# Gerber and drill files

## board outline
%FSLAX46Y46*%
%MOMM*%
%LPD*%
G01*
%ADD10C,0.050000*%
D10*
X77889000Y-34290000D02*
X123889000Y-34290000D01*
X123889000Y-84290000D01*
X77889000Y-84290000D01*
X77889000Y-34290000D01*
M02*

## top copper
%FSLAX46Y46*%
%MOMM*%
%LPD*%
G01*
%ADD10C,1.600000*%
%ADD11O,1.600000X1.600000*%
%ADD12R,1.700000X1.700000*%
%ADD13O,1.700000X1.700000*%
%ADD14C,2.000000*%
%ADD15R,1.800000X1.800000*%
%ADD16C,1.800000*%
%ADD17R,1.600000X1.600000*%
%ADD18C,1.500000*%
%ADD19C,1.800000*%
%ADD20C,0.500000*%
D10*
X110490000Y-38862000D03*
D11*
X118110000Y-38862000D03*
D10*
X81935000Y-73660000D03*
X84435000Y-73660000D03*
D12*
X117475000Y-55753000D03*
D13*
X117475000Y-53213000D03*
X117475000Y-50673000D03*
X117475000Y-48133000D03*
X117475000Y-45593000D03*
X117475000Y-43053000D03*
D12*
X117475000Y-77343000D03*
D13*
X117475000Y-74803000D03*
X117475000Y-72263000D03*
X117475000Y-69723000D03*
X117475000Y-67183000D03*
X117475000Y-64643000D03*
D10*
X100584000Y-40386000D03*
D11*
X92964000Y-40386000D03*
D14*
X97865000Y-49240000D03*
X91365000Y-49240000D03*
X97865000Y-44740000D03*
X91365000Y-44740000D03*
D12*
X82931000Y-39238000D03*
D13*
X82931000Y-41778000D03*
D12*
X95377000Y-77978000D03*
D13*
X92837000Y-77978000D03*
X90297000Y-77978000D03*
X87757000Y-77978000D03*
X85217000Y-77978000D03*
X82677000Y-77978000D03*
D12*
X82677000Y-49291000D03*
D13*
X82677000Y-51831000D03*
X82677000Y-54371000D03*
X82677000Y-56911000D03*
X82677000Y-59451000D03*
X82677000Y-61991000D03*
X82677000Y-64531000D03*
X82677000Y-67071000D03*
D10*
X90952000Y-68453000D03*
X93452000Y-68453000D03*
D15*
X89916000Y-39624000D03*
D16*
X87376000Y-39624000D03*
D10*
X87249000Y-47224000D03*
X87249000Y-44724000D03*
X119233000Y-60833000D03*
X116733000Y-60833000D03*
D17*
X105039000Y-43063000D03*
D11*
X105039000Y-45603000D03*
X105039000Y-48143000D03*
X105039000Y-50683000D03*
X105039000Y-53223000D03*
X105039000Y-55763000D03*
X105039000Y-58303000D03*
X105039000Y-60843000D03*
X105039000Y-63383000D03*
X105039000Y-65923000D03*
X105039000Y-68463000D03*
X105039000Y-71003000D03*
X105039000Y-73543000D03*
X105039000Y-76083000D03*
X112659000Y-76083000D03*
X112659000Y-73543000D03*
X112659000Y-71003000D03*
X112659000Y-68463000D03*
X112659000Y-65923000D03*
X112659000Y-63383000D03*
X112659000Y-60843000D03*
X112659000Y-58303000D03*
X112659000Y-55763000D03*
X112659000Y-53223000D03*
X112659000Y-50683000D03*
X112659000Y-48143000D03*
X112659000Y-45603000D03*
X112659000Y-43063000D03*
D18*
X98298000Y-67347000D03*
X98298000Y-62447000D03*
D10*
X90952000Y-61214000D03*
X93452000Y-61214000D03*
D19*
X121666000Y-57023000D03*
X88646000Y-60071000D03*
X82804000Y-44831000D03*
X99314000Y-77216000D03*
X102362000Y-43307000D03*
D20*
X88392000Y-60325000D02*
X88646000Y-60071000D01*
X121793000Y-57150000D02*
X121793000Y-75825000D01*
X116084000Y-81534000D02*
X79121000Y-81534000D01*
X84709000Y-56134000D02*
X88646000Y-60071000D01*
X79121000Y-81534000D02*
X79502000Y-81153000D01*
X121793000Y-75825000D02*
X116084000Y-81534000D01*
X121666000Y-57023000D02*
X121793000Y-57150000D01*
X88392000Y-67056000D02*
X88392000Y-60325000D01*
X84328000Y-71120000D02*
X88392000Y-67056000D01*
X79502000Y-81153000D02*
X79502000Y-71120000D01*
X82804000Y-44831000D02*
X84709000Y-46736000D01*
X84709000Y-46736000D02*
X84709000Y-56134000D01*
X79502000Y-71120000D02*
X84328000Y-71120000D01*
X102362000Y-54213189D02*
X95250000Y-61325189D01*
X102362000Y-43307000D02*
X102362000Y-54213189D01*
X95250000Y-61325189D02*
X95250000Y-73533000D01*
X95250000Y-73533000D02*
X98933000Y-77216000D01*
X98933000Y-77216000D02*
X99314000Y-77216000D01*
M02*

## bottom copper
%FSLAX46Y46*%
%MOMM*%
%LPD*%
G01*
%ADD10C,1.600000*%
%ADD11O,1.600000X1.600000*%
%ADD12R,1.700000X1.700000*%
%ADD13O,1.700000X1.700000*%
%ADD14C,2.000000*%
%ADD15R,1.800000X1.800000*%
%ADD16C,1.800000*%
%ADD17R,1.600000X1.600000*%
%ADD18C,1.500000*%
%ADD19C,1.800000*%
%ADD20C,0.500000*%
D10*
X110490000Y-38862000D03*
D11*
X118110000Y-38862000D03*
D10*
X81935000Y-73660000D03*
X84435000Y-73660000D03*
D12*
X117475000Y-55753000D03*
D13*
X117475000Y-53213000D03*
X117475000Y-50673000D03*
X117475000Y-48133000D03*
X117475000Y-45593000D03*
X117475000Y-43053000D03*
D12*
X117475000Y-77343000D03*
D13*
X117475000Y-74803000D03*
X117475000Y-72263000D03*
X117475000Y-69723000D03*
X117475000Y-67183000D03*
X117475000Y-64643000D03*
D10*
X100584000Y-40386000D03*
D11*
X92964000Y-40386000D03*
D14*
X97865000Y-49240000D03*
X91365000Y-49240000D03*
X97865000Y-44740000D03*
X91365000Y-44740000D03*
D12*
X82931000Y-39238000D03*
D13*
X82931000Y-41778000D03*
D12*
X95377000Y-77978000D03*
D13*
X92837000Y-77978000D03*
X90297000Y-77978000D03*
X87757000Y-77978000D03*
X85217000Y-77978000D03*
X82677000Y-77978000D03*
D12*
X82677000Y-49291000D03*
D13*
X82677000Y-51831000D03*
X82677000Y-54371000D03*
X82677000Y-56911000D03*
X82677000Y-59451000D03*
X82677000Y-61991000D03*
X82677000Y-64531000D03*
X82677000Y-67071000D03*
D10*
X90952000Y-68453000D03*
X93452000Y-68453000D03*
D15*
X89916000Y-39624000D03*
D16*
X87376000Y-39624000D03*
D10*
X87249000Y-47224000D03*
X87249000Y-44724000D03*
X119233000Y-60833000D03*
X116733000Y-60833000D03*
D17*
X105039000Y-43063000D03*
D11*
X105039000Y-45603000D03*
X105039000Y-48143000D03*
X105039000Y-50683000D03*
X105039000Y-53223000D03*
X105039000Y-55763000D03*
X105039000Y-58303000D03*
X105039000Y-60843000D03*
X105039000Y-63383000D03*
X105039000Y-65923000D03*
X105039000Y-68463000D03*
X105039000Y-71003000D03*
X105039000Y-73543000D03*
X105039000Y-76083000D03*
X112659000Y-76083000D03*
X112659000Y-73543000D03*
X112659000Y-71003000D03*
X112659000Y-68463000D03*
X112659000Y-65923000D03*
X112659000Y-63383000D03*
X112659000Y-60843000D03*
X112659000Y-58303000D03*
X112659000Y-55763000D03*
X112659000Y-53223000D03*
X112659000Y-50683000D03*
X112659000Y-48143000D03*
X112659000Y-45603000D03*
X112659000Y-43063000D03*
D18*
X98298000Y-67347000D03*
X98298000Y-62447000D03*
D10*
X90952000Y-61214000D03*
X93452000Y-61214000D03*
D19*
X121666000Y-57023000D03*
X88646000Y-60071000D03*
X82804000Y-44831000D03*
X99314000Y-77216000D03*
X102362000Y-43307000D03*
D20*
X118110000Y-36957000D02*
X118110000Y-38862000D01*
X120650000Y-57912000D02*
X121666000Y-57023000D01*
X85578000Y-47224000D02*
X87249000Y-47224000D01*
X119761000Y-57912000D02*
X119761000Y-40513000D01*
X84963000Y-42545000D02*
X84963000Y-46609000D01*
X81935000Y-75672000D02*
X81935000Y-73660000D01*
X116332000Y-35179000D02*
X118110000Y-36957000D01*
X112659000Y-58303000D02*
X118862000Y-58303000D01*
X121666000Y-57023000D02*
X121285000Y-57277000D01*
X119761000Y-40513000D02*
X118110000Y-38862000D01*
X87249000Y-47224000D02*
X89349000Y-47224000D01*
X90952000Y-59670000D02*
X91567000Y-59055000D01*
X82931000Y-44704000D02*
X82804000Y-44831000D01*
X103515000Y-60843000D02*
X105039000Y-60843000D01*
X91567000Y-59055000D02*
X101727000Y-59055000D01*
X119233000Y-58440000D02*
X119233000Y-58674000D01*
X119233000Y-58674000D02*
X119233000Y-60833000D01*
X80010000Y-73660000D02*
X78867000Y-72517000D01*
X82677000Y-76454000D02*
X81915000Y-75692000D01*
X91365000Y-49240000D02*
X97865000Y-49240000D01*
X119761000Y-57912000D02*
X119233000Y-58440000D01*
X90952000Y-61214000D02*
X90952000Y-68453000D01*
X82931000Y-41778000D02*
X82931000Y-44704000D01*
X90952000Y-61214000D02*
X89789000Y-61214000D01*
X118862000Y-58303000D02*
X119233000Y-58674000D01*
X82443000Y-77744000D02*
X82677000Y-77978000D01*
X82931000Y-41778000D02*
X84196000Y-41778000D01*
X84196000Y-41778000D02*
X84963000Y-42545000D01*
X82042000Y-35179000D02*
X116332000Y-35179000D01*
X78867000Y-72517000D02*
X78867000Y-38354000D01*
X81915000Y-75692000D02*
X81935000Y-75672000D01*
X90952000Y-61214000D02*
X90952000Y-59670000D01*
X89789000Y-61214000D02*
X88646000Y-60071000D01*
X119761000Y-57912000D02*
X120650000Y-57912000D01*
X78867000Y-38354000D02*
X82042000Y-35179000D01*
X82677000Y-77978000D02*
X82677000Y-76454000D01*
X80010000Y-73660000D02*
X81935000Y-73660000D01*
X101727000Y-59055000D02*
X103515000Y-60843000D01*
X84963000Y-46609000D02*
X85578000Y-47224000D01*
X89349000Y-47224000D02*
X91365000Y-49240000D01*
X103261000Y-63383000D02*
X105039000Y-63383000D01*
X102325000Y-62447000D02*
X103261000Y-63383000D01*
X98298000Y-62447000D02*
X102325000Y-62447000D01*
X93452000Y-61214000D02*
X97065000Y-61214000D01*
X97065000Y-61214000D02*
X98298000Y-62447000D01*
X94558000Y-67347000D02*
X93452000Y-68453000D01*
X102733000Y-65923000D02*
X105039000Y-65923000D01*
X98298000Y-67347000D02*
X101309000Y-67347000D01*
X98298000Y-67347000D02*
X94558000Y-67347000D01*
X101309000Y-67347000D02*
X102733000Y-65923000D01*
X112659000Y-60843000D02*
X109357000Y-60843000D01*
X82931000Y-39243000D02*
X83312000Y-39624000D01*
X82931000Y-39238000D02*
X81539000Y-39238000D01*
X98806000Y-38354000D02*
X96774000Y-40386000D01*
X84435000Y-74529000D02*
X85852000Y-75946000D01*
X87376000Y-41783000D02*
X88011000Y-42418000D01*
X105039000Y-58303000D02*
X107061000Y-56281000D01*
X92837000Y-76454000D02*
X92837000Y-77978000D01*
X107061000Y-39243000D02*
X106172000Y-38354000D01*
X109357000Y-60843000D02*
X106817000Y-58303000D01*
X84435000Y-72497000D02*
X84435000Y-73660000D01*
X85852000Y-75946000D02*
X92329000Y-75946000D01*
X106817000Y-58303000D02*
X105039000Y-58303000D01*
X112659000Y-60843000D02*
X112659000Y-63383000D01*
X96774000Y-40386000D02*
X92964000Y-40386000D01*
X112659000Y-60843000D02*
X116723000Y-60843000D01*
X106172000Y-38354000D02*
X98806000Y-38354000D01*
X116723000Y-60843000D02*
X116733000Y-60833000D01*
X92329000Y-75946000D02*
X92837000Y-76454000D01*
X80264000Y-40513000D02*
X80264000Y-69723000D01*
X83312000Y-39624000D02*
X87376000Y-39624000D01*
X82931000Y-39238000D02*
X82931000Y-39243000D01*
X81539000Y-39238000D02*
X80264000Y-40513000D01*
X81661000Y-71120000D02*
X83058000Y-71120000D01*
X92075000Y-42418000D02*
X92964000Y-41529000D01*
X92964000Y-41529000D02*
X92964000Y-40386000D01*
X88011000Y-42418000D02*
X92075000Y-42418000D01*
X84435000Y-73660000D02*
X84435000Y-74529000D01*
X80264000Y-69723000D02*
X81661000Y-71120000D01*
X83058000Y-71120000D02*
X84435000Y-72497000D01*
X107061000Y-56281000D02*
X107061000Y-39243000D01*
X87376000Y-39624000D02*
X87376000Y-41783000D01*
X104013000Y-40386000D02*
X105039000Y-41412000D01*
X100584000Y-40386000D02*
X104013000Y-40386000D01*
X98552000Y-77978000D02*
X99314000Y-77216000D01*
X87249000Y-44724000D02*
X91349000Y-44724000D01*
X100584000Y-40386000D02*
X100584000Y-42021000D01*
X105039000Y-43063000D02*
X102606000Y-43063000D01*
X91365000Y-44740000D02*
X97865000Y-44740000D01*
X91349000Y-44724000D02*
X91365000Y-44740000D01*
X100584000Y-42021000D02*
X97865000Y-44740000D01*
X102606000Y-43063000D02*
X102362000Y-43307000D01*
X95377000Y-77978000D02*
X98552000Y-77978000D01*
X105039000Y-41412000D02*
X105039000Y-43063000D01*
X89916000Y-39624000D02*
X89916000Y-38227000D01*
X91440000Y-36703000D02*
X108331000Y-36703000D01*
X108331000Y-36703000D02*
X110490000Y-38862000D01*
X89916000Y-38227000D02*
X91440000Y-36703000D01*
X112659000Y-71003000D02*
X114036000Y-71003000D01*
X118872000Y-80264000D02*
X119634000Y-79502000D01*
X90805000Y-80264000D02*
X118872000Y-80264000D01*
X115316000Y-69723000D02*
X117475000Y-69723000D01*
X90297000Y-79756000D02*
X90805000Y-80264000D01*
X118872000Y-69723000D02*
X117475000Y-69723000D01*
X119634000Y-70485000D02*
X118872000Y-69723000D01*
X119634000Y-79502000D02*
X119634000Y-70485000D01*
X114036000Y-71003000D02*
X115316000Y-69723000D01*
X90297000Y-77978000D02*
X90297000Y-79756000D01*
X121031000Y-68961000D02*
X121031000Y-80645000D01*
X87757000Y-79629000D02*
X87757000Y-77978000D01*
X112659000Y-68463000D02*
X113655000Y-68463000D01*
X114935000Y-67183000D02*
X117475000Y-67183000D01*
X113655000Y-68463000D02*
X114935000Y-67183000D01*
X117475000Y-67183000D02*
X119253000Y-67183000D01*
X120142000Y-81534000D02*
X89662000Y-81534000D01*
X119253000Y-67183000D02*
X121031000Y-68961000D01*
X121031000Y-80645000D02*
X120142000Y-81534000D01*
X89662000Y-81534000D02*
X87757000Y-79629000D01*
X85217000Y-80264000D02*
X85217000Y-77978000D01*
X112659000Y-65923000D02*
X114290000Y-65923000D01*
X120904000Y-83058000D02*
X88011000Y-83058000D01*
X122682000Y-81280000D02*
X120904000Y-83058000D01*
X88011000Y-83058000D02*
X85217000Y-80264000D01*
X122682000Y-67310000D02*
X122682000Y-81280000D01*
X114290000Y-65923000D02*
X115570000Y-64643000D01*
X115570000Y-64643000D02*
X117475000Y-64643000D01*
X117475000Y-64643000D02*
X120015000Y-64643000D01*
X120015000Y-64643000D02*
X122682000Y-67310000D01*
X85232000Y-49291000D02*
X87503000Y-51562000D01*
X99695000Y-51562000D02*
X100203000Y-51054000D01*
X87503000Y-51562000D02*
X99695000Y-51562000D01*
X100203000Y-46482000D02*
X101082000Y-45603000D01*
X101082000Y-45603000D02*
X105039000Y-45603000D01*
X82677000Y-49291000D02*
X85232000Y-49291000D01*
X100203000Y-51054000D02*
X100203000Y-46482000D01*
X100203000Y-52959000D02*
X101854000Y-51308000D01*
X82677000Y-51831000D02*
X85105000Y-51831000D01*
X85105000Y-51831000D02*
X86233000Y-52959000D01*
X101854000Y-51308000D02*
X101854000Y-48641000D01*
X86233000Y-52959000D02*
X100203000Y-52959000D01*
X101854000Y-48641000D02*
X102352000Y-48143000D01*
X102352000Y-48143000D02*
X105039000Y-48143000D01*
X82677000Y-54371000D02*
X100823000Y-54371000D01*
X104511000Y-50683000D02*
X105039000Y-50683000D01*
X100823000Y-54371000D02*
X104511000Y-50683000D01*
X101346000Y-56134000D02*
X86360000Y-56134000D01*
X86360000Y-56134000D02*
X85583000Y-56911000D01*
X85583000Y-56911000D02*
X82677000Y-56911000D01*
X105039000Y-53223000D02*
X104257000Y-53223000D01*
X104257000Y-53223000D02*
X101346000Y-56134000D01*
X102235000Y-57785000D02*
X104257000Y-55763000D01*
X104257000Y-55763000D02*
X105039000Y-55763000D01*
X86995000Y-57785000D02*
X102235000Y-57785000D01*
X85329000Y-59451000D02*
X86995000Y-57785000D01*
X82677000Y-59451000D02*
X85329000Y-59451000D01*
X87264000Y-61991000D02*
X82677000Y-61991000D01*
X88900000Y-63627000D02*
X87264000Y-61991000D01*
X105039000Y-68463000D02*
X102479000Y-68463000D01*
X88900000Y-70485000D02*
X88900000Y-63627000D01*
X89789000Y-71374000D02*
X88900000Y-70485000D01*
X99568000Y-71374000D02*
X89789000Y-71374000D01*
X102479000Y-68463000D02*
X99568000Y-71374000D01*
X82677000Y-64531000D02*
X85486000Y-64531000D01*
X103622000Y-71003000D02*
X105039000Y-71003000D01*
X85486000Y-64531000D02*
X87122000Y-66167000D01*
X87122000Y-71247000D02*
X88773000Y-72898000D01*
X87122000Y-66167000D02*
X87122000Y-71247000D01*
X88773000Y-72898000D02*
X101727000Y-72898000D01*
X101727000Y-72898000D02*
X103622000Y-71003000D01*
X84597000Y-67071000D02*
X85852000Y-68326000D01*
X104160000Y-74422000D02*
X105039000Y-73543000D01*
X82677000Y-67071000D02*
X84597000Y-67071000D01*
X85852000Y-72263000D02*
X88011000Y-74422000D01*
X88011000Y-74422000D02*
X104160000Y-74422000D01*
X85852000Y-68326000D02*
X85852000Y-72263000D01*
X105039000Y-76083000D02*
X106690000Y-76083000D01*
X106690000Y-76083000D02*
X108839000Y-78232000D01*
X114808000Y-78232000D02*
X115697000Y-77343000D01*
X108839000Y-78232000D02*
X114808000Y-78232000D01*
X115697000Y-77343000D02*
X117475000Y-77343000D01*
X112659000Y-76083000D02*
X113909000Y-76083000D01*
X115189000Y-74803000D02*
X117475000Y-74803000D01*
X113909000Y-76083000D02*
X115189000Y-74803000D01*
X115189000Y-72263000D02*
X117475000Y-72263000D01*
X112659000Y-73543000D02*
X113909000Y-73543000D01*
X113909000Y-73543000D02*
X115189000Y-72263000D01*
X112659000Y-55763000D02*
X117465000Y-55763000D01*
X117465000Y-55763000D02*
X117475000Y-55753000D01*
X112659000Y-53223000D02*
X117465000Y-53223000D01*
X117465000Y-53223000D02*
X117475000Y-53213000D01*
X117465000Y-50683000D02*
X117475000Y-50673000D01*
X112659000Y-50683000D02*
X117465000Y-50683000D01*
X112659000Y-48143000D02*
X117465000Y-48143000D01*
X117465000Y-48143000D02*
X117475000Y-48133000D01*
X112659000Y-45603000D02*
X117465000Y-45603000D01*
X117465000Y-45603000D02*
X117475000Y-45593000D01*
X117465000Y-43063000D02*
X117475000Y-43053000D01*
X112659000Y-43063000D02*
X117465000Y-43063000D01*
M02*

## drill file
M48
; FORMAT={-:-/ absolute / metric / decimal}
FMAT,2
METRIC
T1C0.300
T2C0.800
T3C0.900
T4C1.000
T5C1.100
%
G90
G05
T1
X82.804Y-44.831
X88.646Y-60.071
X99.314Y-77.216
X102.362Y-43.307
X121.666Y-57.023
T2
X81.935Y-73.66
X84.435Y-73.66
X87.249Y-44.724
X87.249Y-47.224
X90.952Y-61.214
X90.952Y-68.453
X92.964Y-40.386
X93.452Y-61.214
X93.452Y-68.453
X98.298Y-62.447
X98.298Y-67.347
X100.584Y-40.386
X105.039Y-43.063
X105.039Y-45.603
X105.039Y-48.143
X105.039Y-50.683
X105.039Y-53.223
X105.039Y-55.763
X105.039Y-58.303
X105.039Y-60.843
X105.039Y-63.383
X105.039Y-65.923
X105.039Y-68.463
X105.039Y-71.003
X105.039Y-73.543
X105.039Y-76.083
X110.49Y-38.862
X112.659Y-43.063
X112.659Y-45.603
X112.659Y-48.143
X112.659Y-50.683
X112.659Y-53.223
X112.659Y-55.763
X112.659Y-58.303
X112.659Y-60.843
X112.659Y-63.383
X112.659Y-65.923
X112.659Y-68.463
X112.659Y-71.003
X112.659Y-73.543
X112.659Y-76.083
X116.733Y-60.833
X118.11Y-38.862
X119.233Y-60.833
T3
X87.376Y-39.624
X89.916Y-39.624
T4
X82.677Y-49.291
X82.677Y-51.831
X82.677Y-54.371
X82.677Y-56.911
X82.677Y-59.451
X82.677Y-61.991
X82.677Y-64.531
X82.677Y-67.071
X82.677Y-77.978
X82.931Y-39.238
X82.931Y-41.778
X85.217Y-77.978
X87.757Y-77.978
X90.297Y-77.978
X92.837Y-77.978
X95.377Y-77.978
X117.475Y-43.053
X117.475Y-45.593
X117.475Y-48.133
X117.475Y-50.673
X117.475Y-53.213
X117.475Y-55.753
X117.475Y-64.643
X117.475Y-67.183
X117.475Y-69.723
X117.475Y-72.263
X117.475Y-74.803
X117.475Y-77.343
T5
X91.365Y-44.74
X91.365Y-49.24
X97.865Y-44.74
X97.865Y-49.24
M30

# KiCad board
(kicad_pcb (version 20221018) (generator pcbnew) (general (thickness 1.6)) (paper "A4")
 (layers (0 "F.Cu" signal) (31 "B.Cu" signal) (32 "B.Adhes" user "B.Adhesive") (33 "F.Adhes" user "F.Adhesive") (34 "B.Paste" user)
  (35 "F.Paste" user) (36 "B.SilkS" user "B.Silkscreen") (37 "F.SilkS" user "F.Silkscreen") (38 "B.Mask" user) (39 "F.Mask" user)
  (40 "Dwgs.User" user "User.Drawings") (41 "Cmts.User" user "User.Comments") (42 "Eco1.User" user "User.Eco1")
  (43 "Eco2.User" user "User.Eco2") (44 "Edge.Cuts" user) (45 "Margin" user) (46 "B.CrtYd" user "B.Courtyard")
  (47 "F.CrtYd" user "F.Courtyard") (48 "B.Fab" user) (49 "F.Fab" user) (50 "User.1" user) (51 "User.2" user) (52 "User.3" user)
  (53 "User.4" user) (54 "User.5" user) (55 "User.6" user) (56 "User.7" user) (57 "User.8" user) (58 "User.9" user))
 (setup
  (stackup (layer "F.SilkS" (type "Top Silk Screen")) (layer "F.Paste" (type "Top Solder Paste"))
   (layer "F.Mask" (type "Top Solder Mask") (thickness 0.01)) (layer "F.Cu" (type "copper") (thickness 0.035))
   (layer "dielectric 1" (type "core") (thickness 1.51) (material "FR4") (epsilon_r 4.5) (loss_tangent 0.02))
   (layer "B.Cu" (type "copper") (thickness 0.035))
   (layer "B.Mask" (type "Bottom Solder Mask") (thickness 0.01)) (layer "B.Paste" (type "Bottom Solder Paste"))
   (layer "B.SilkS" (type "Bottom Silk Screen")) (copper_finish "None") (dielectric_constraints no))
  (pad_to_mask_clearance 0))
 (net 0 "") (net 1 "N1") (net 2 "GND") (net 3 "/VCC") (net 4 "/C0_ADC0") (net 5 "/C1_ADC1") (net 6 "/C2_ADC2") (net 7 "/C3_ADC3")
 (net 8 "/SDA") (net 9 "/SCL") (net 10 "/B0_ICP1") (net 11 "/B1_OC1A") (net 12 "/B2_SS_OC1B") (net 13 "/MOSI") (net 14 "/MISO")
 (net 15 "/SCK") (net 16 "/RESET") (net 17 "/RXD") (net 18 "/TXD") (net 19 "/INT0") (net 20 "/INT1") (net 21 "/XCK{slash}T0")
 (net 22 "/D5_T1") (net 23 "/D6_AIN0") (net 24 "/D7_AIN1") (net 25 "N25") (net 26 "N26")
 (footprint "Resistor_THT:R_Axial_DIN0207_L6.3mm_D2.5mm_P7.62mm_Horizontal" (layer "F.Cu") (at 110.49 38.862)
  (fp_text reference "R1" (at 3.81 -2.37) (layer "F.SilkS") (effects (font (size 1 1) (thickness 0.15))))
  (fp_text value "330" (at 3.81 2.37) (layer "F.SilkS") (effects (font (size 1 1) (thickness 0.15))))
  (pad "1" thru_hole circle (at 0 0) (size 1.6 1.6) (drill 0.8) (layers "*.Cu" "*.Mask") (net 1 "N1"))
  (pad "2" thru_hole oval (at 7.62 0) (size 1.6 1.6) (drill 0.8) (layers "*.Cu" "*.Mask") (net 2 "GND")))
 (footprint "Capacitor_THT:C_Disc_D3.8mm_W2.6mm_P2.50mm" (layer "F.Cu") (at 81.935 73.66)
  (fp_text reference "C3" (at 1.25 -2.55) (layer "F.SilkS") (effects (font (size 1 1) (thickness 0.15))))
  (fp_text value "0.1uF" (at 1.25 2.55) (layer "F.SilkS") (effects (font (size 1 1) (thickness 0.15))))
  (pad "1" thru_hole circle (at 0 0) (size 1.6 1.6) (drill 0.8) (layers "*.Cu" "*.Mask") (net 2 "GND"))
  (pad "2" thru_hole circle (at 2.5 0) (size 1.6 1.6) (drill 0.8) (layers "*.Cu" "*.Mask") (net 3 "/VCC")))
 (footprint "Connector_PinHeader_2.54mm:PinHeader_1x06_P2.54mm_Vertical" (layer "F.Cu") (at 117.475 55.753 180)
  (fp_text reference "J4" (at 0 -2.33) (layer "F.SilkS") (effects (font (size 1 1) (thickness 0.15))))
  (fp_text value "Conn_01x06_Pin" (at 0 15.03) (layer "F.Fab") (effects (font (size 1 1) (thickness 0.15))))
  (pad "1" thru_hole rect (at 0 0 180) (size 1.7 1.7) (drill 1) (layers "*.Cu" "*.Mask") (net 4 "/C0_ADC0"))
  (pad "2" thru_hole oval (at 0 2.54 180) (size 1.7 1.7) (drill 1) (layers "*.Cu" "*.Mask") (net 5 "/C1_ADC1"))
  (pad "3" thru_hole oval (at 0 5.08 180) (size 1.7 1.7) (drill 1) (layers "*.Cu" "*.Mask") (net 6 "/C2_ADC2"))
  (pad "4" thru_hole oval (at 0 7.62 180) (size 1.7 1.7) (drill 1) (layers "*.Cu" "*.Mask") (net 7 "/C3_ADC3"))
  (pad "5" thru_hole oval (at 0 10.16 180) (size 1.7 1.7) (drill 1) (layers "*.Cu" "*.Mask") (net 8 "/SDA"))
  (pad "6" thru_hole oval (at 0 12.7 180) (size 1.7 1.7) (drill 1) (layers "*.Cu" "*.Mask") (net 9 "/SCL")))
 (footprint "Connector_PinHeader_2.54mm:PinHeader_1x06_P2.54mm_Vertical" (layer "F.Cu") (at 117.475 77.343 180)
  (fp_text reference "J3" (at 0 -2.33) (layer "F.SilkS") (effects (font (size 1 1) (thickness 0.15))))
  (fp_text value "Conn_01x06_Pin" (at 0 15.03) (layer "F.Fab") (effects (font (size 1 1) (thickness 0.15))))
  (pad "1" thru_hole rect (at 0 0 180) (size 1.7 1.7) (drill 1) (layers "*.Cu" "*.Mask") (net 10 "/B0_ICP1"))
  (pad "2" thru_hole oval (at 0 2.54 180) (size 1.7 1.7) (drill 1) (layers "*.Cu" "*.Mask") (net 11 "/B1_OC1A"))
  (pad "3" thru_hole oval (at 0 5.08 180) (size 1.7 1.7) (drill 1) (layers "*.Cu" "*.Mask") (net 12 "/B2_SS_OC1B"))
  (pad "4" thru_hole oval (at 0 7.62 180) (size 1.7 1.7) (drill 1) (layers "*.Cu" "*.Mask") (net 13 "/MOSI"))
  (pad "5" thru_hole oval (at 0 10.16 180) (size 1.7 1.7) (drill 1) (layers "*.Cu" "*.Mask") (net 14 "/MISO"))
  (pad "6" thru_hole oval (at 0 12.7 180) (size 1.7 1.7) (drill 1) (layers "*.Cu" "*.Mask") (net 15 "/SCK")))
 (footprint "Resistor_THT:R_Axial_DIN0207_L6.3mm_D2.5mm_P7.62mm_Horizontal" (layer "F.Cu") (at 100.584 40.386 180)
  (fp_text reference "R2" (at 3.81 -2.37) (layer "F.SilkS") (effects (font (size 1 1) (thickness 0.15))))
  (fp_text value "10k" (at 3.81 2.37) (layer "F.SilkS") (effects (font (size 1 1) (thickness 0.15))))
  (pad "1" thru_hole circle (at 0 0 180) (size 1.6 1.6) (drill 0.8) (layers "*.Cu" "*.Mask") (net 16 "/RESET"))
  (pad "2" thru_hole oval (at 7.62 0 180) (size 1.6 1.6) (drill 0.8) (layers "*.Cu" "*.Mask") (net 3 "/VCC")))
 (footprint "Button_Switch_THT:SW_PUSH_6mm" (layer "F.Cu") (at 97.865 49.24 180)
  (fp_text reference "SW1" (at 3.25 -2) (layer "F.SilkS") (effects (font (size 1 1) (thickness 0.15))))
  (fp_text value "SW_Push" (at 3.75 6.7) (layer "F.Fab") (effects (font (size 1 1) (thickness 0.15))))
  (pad "1" thru_hole circle (at 0 0 270) (size 2 2) (drill 1.1) (layers "*.Cu" "*.Mask") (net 2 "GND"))
  (pad "1" thru_hole circle (at 6.5 0 270) (size 2 2) (drill 1.1) (layers "*.Cu" "*.Mask") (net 2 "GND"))
  (pad "2" thru_hole circle (at 0 4.5 270) (size 2 2) (drill 1.1) (layers "*.Cu" "*.Mask") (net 16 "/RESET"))
  (pad "2" thru_hole circle (at 6.5 4.5 270) (size 2 2) (drill 1.1) (layers "*.Cu" "*.Mask") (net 16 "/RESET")))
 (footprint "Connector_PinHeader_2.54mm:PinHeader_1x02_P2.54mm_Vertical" (layer "F.Cu") (at 82.931 39.238)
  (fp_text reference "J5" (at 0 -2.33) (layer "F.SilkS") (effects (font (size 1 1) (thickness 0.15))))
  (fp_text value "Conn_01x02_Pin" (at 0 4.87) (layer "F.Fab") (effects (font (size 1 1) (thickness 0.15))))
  (pad "1" thru_hole rect (at 0 0) (size 1.7 1.7) (drill 1) (layers "*.Cu" "*.Mask") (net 3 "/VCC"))
  (pad "2" thru_hole oval (at 0 2.54) (size 1.7 1.7) (drill 1) (layers "*.Cu" "*.Mask") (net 2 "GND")))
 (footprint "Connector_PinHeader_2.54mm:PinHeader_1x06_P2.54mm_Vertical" (layer "F.Cu") (at 95.377 77.978 -90)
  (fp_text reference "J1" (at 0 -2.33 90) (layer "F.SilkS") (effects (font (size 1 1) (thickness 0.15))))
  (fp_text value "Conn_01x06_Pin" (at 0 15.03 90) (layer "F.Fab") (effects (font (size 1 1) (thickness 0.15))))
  (pad "1" thru_hole rect (at 0 0 270) (size 1.7 1.7) (drill 1) (layers "*.Cu" "*.Mask") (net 16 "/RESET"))
  (pad "2" thru_hole oval (at 0 2.54 270) (size 1.7 1.7) (drill 1) (layers "*.Cu" "*.Mask") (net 3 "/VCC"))
  (pad "3" thru_hole oval (at 0 5.08 270) (size 1.7 1.7) (drill 1) (layers "*.Cu" "*.Mask") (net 13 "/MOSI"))
  (pad "4" thru_hole oval (at 0 7.62 270) (size 1.7 1.7) (drill 1) (layers "*.Cu" "*.Mask") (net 14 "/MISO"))
  (pad "5" thru_hole oval (at 0 10.16 270) (size 1.7 1.7) (drill 1) (layers "*.Cu" "*.Mask") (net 15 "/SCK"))
  (pad "6" thru_hole oval (at 0 12.7 270) (size 1.7 1.7) (drill 1) (layers "*.Cu" "*.Mask") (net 2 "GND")))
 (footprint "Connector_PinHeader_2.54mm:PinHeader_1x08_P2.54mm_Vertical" (layer "F.Cu") (at 82.677 49.291)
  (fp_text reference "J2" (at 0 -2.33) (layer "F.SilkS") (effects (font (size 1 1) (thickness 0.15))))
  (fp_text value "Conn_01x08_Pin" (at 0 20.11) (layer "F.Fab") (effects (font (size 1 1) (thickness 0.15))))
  (pad "1" thru_hole rect (at 0 0) (size 1.7 1.7) (drill 1) (layers "*.Cu" "*.Mask") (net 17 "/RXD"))
  (pad "2" thru_hole oval (at 0 2.54) (size 1.7 1.7) (drill 1) (layers "*.Cu" "*.Mask") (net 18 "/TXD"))
  (pad "3" thru_hole oval (at 0 5.08) (size 1.7 1.7) (drill 1) (layers "*.Cu" "*.Mask") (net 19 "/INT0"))
  (pad "4" thru_hole oval (at 0 7.62) (size 1.7 1.7) (drill 1) (layers "*.Cu" "*.Mask") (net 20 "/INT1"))
  (pad "5" thru_hole oval (at 0 10.16) (size 1.7 1.7) (drill 1) (layers "*.Cu" "*.Mask") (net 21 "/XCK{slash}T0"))
  (pad "6" thru_hole oval (at 0 12.7) (size 1.7 1.7) (drill 1) (layers "*.Cu" "*.Mask") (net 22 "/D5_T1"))
  (pad "7" thru_hole oval (at 0 15.24) (size 1.7 1.7) (drill 1) (layers "*.Cu" "*.Mask") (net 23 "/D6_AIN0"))
  (pad "8" thru_hole oval (at 0 17.78) (size 1.7 1.7) (drill 1) (layers "*.Cu" "*.Mask") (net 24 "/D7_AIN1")))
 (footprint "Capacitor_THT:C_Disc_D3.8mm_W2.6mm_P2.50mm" (layer "F.Cu") (at 90.952 68.453)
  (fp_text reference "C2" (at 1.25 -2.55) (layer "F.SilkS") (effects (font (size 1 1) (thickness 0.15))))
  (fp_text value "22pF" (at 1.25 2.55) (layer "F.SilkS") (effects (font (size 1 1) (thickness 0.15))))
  (pad "1" thru_hole circle (at 0 0) (size 1.6 1.6) (drill 0.8) (layers "*.Cu" "*.Mask") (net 2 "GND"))
  (pad "2" thru_hole circle (at 2.5 0) (size 1.6 1.6) (drill 0.8) (layers "*.Cu" "*.Mask") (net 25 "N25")))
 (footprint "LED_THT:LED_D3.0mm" (layer "F.Cu") (at 89.916 39.624 180)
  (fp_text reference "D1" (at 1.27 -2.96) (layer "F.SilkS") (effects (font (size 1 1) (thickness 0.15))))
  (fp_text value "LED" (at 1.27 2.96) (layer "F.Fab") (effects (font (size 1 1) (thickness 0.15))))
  (pad "1" thru_hole rect (at 0 0 180) (size 1.8 1.8) (drill 0.9) (layers "*.Cu" "*.Mask") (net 1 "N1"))
  (pad "2" thru_hole circle (at 2.54 0 180) (size 1.8 1.8) (drill 0.9) (layers "*.Cu" "*.Mask") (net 3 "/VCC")))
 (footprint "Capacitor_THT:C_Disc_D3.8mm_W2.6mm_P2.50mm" (layer "F.Cu") (at 87.249 47.224 90)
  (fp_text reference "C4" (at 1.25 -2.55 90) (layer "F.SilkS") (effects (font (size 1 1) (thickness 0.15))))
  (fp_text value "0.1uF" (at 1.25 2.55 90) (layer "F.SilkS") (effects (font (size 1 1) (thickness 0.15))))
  (pad "1" thru_hole circle (at 0 0 90) (size 1.6 1.6) (drill 0.8) (layers "*.Cu" "*.Mask") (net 2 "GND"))
  (pad "2" thru_hole circle (at 2.5 0 90) (size 1.6 1.6) (drill 0.8) (layers "*.Cu" "*.Mask") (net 16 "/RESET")))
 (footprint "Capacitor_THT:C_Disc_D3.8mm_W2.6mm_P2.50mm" (layer "F.Cu") (at 119.233 60.833 180)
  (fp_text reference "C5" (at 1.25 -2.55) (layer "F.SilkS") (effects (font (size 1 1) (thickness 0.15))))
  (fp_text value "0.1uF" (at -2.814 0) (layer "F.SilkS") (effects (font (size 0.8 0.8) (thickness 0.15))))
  (pad "1" thru_hole circle (at 0 0 180) (size 1.6 1.6) (drill 0.8) (layers "*.Cu" "*.Mask") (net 2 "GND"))
  (pad "2" thru_hole circle (at 2.5 0 180) (size 1.6 1.6) (drill 0.8) (layers "*.Cu" "*.Mask") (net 3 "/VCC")))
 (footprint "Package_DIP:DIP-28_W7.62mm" (layer "F.Cu") (at 105.039 43.063)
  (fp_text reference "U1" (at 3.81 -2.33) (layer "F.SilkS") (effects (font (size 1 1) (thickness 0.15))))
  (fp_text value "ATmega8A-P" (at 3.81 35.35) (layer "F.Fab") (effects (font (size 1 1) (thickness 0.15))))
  (pad "1" thru_hole rect (at 0 0) (size 1.6 1.6) (drill 0.8) (layers "*.Cu" "*.Mask") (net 16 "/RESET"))
  (pad "2" thru_hole oval (at 0 2.54) (size 1.6 1.6) (drill 0.8) (layers "*.Cu" "*.Mask") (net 17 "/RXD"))
  (pad "3" thru_hole oval (at 0 5.08) (size 1.6 1.6) (drill 0.8) (layers "*.Cu" "*.Mask") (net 18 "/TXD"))
  (pad "4" thru_hole oval (at 0 7.62) (size 1.6 1.6) (drill 0.8) (layers "*.Cu" "*.Mask") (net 19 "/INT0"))
  (pad "5" thru_hole oval (at 0 10.16) (size 1.6 1.6) (drill 0.8) (layers "*.Cu" "*.Mask") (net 20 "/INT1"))
  (pad "6" thru_hole oval (at 0 12.7) (size 1.6 1.6) (drill 0.8) (layers "*.Cu" "*.Mask") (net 21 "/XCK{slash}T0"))
  (pad "7" thru_hole oval (at 0 15.24) (size 1.6 1.6) (drill 0.8) (layers "*.Cu" "*.Mask") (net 3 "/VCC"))
  (pad "8" thru_hole oval (at 0 17.78) (size 1.6 1.6) (drill 0.8) (layers "*.Cu" "*.Mask") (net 2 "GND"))
  (pad "9" thru_hole oval (at 0 20.32) (size 1.6 1.6) (drill 0.8) (layers "*.Cu" "*.Mask") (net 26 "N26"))
  (pad "10" thru_hole oval (at 0 22.86) (size 1.6 1.6) (drill 0.8) (layers "*.Cu" "*.Mask") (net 25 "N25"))
  (pad "11" thru_hole oval (at 0 25.4) (size 1.6 1.6) (drill 0.8) (layers "*.Cu" "*.Mask") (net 22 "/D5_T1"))
  (pad "12" thru_hole oval (at 0 27.94) (size 1.6 1.6) (drill 0.8) (layers "*.Cu" "*.Mask") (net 23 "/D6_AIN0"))
  (pad "13" thru_hole oval (at 0 30.48) (size 1.6 1.6) (drill 0.8) (layers "*.Cu" "*.Mask") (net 24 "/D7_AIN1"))
  (pad "14" thru_hole oval (at 0 33.02) (size 1.6 1.6) (drill 0.8) (layers "*.Cu" "*.Mask") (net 10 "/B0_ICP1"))
  (pad "15" thru_hole oval (at 7.62 33.02) (size 1.6 1.6) (drill 0.8) (layers "*.Cu" "*.Mask") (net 11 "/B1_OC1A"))
  (pad "16" thru_hole oval (at 7.62 30.48) (size 1.6 1.6) (drill 0.8) (layers "*.Cu" "*.Mask") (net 12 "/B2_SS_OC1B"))
  (pad "17" thru_hole oval (at 7.62 27.94) (size 1.6 1.6) (drill 0.8) (layers "*.Cu" "*.Mask") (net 13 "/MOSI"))
  (pad "18" thru_hole oval (at 7.62 25.4) (size 1.6 1.6) (drill 0.8) (layers "*.Cu" "*.Mask") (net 14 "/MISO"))
  (pad "19" thru_hole oval (at 7.62 22.86) (size 1.6 1.6) (drill 0.8) (layers "*.Cu" "*.Mask") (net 15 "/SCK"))
  (pad "20" thru_hole oval (at 7.62 20.32) (size 1.6 1.6) (drill 0.8) (layers "*.Cu" "*.Mask") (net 3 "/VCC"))
  (pad "21" thru_hole oval (at 7.62 17.78) (size 1.6 1.6) (drill 0.8) (layers "*.Cu" "*.Mask") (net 3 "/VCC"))
  (pad "22" thru_hole oval (at 7.62 15.24) (size 1.6 1.6) (drill 0.8) (layers "*.Cu" "*.Mask") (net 2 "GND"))
  (pad "23" thru_hole oval (at 7.62 12.7) (size 1.6 1.6) (drill 0.8) (layers "*.Cu" "*.Mask") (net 4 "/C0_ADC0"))
  (pad "24" thru_hole oval (at 7.62 10.16) (size 1.6 1.6) (drill 0.8) (layers "*.Cu" "*.Mask") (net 5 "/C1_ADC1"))
  (pad "25" thru_hole oval (at 7.62 7.62) (size 1.6 1.6) (drill 0.8) (layers "*.Cu" "*.Mask") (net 6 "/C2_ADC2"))
  (pad "26" thru_hole oval (at 7.62 5.08) (size 1.6 1.6) (drill 0.8) (layers "*.Cu" "*.Mask") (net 7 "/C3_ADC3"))
  (pad "27" thru_hole oval (at 7.62 2.54) (size 1.6 1.6) (drill 0.8) (layers "*.Cu" "*.Mask") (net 8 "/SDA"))
  (pad "28" thru_hole oval (at 7.62 0) (size 1.6 1.6) (drill 0.8) (layers "*.Cu" "*.Mask") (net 9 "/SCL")))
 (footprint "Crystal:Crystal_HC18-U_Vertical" (layer "F.Cu") (at 98.298 67.347 90)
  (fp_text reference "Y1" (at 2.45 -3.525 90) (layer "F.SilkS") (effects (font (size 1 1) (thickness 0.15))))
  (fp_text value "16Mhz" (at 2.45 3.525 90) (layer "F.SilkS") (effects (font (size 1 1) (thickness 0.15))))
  (pad "1" thru_hole circle (at 0 0 90) (size 1.5 1.5) (drill 0.8) (layers "*.Cu" "*.Mask") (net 25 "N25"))
  (pad "2" thru_hole circle (at 4.9 0 90) (size 1.5 1.5) (drill 0.8) (layers "*.Cu" "*.Mask") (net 26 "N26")))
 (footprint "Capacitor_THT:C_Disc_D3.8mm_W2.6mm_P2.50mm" (layer "F.Cu") (at 90.952 61.214)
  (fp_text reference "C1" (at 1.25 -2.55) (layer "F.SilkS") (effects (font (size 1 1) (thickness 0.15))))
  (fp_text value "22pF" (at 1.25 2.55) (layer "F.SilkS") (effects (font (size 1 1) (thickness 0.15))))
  (pad "1" thru_hole circle (at 0 0) (size 1.6 1.6) (drill 0.8) (layers "*.Cu" "*.Mask") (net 2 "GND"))
  (pad "2" thru_hole circle (at 2.5 0) (size 1.6 1.6) (drill 0.8) (layers "*.Cu" "*.Mask") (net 26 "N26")))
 (gr_rect (start 77.889 34.29) (end 123.889 84.29) (stroke (width 0.05) (type default)) (fill none) (layer "Edge.Cuts"))
 (segment (start 88.392 60.325) (end 88.646 60.071) (width 0.5) (layer "F.Cu") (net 2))
 (segment (start 121.793 57.15) (end 121.793 75.825) (width 0.5) (layer "F.Cu") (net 2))
 (segment (start 116.084 81.534) (end 79.121 81.534) (width 0.5) (layer "F.Cu") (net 2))
 (segment (start 84.709 56.134) (end 88.646 60.071) (width 0.5) (layer "F.Cu") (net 2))
 (segment (start 79.121 81.534) (end 79.502 81.153) (width 0.5) (layer "F.Cu") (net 2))
 (segment (start 121.793 75.825) (end 116.084 81.534) (width 0.5) (layer "F.Cu") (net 2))
 (segment (start 121.666 57.023) (end 121.793 57.15) (width 0.5) (layer "F.Cu") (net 2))
 (segment (start 88.392 67.056) (end 88.392 60.325) (width 0.5) (layer "F.Cu") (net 2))
 (segment (start 84.328 71.12) (end 88.392 67.056) (width 0.5) (layer "F.Cu") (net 2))
 (segment (start 79.502 81.153) (end 79.502 71.12) (width 0.5) (layer "F.Cu") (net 2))
 (segment (start 82.804 44.831) (end 84.709 46.736) (width 0.5) (layer "F.Cu") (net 2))
 (segment (start 84.709 46.736) (end 84.709 56.134) (width 0.5) (layer "F.Cu") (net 2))
 (segment (start 79.502 71.12) (end 84.328 71.12) (width 0.5) (layer "F.Cu") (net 2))
 (via (at 121.666 57.023) (size 1.8) (drill 0.3) (layers "F.Cu" "B.Cu") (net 2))
 (via (at 88.646 60.071) (size 1.8) (drill 0.3) (layers "F.Cu" "B.Cu") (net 2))
 (via (at 82.804 44.831) (size 1.8) (drill 0.3) (layers "F.Cu" "B.Cu") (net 2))
 (segment (start 118.11 36.957) (end 118.11 38.862) (width 0.5) (layer "B.Cu") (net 2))
 (segment (start 120.65 57.912) (end 121.666 57.023) (width 0.5) (layer "B.Cu") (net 2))
 (segment (start 85.578 47.224) (end 87.249 47.224) (width 0.5) (layer "B.Cu") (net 2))
 (segment (start 119.761 57.912) (end 119.761 40.513) (width 0.5) (layer "B.Cu") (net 2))
 (segment (start 84.963 42.545) (end 84.963 46.609) (width 0.5) (layer "B.Cu") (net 2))
 (segment (start 81.935 75.672) (end 81.935 73.66) (width 0.5) (layer "B.Cu") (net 2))
 (segment (start 116.332 35.179) (end 118.11 36.957) (width 0.5) (layer "B.Cu") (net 2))
 (segment (start 112.659 58.303) (end 118.862 58.303) (width 0.5) (layer "B.Cu") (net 2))
 (segment (start 121.666 57.023) (end 121.285 57.277) (width 0.5) (layer "B.Cu") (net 2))
 (segment (start 119.761 40.513) (end 118.11 38.862) (width 0.5) (layer "B.Cu") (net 2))
 (segment (start 87.249 47.224) (end 89.349 47.224) (width 0.5) (layer "B.Cu") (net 2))
 (segment (start 90.952 59.67) (end 91.567 59.055) (width 0.5) (layer "B.Cu") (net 2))
 (segment (start 82.931 44.704) (end 82.804 44.831) (width 0.5) (layer "B.Cu") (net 2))
 (segment (start 103.515 60.843) (end 105.039 60.843) (width 0.5) (layer "B.Cu") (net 2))
 (segment (start 91.567 59.055) (end 101.727 59.055) (width 0.5) (layer "B.Cu") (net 2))
 (segment (start 119.233 58.44) (end 119.233 58.674) (width 0.5) (layer "B.Cu") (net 2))
 (segment (start 119.233 58.674) (end 119.233 60.833) (width 0.5) (layer "B.Cu") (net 2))
 (segment (start 80.01 73.66) (end 78.867 72.517) (width 0.5) (layer "B.Cu") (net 2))
 (segment (start 82.677 76.454) (end 81.915 75.692) (width 0.5) (layer "B.Cu") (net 2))
 (segment (start 91.365 49.24) (end 97.865 49.24) (width 0.5) (layer "B.Cu") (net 2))
 (segment (start 119.761 57.912) (end 119.233 58.44) (width 0.5) (layer "B.Cu") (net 2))
 (segment (start 90.952 61.214) (end 90.952 68.453) (width 0.5) (layer "B.Cu") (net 2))
 (segment (start 82.931 41.778) (end 82.931 44.704) (width 0.5) (layer "B.Cu") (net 2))
 (segment (start 90.952 61.214) (end 89.789 61.214) (width 0.5) (layer "B.Cu") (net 2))
 (segment (start 118.862 58.303) (end 119.233 58.674) (width 0.5) (layer "B.Cu") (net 2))
 (segment (start 82.443 77.744) (end 82.677 77.978) (width 0.5) (layer "B.Cu") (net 2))
 (segment (start 82.931 41.778) (end 84.196 41.778) (width 0.5) (layer "B.Cu") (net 2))
 (segment (start 84.196 41.778) (end 84.963 42.545) (width 0.5) (layer "B.Cu") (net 2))
 (segment (start 82.042 35.179) (end 116.332 35.179) (width 0.5) (layer "B.Cu") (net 2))
 (segment (start 78.867 72.517) (end 78.867 38.354) (width 0.5) (layer "B.Cu") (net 2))
 (segment (start 81.915 75.692) (end 81.935 75.672) (width 0.5) (layer "B.Cu") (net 2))
 (segment (start 90.952 61.214) (end 90.952 59.67) (width 0.5) (layer "B.Cu") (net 2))
 (segment (start 89.789 61.214) (end 88.646 60.071) (width 0.5) (layer "B.Cu") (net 2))
 (segment (start 119.761 57.912) (end 120.65 57.912) (width 0.5) (layer "B.Cu") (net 2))
 (segment (start 78.867 38.354) (end 82.042 35.179) (width 0.5) (layer "B.Cu") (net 2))
 (segment (start 82.677 77.978) (end 82.677 76.454) (width 0.5) (layer "B.Cu") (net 2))
 (segment (start 80.01 73.66) (end 81.935 73.66) (width 0.5) (layer "B.Cu") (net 2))
 (segment (start 101.727 59.055) (end 103.515 60.843) (width 0.5) (layer "B.Cu") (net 2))
 (segment (start 84.963 46.609) (end 85.578 47.224) (width 0.5) (layer "B.Cu") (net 2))
 (segment (start 89.349 47.224) (end 91.365 49.24) (width 0.5) (layer "B.Cu") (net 2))
 (segment (start 103.261 63.383) (end 105.039 63.383) (width 0.5) (layer "B.Cu") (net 26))
 (segment (start 102.325 62.447) (end 103.261 63.383) (width 0.5) (layer "B.Cu") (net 26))
 (segment (start 98.298 62.447) (end 102.325 62.447) (width 0.5) (layer "B.Cu") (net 26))
 (segment (start 93.452 61.214) (end 97.065 61.214) (width 0.5) (layer "B.Cu") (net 26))
 (segment (start 97.065 61.214) (end 98.298 62.447) (width 0.5) (layer "B.Cu") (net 26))
 (segment (start 94.558 67.347) (end 93.452 68.453) (width 0.5) (layer "B.Cu") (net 25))
 (segment (start 102.733 65.923) (end 105.039 65.923) (width 0.5) (layer "B.Cu") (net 25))
 (segment (start 98.298 67.347) (end 101.309 67.347) (width 0.5) (layer "B.Cu") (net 25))
 (segment (start 98.298 67.347) (end 94.558 67.347) (width 0.5) (layer "B.Cu") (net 25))
 (segment (start 101.309 67.347) (end 102.733 65.923) (width 0.5) (layer "B.Cu") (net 25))
 (segment (start 112.659 60.843) (end 109.357 60.843) (width 0.5) (layer "B.Cu") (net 3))
 (segment (start 82.931 39.243) (end 83.312 39.624) (width 0.5) (layer "B.Cu") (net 3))
 (segment (start 82.931 39.238) (end 81.539 39.238) (width 0.5) (layer "B.Cu") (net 3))
 (segment (start 98.806 38.354) (end 96.774 40.386) (width 0.5) (layer "B.Cu") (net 3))
 (segment (start 84.435 74.529) (end 85.852 75.946) (width 0.5) (layer "B.Cu") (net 3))
 (segment (start 87.376 41.783) (end 88.011 42.418) (width 0.5) (layer "B.Cu") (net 3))
 (segment (start 105.039 58.303) (end 107.061 56.281) (width 0.5) (layer "B.Cu") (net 3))
 (segment (start 92.837 76.454) (end 92.837 77.978) (width 0.5) (layer "B.Cu") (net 3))
 (segment (start 107.061 39.243) (end 106.172 38.354) (width 0.5) (layer "B.Cu") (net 3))
 (segment (start 109.357 60.843) (end 106.817 58.303) (width 0.5) (layer "B.Cu") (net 3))
 (segment (start 84.435 72.497) (end 84.435 73.66) (width 0.5) (layer "B.Cu") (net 3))
 (segment (start 85.852 75.946) (end 92.329 75.946) (width 0.5) (layer "B.Cu") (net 3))
 (segment (start 106.817 58.303) (end 105.039 58.303) (width 0.5) (layer "B.Cu") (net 3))
 (segment (start 112.659 60.843) (end 112.659 63.383) (width 0.5) (layer "B.Cu") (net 3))
 (segment (start 96.774 40.386) (end 92.964 40.386) (width 0.5) (layer "B.Cu") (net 3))
 (segment (start 112.659 60.843) (end 116.723 60.843) (width 0.5) (layer "B.Cu") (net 3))
 (segment (start 106.172 38.354) (end 98.806 38.354) (width 0.5) (layer "B.Cu") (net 3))
 (segment (start 116.723 60.843) (end 116.733 60.833) (width 0.5) (layer "B.Cu") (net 3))
 (segment (start 92.329 75.946) (end 92.837 76.454) (width 0.5) (layer "B.Cu") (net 3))
 (segment (start 80.264 40.513) (end 80.264 69.723) (width 0.5) (layer "B.Cu") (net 3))
 (segment (start 83.312 39.624) (end 87.376 39.624) (width 0.5) (layer "B.Cu") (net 3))
 (segment (start 82.931 39.238) (end 82.931 39.243) (width 0.5) (layer "B.Cu") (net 3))
 (segment (start 81.539 39.238) (end 80.264 40.513) (width 0.5) (layer "B.Cu") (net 3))
 (segment (start 81.661 71.12) (end 83.058 71.12) (width 0.5) (layer "B.Cu") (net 3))
 (segment (start 92.075 42.418) (end 92.964 41.529) (width 0.5) (layer "B.Cu") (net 3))
 (segment (start 92.964 41.529) (end 92.964 40.386) (width 0.5) (layer "B.Cu") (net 3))
 (segment (start 88.011 42.418) (end 92.075 42.418) (width 0.5) (layer "B.Cu") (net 3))
 (segment (start 84.435 73.66) (end 84.435 74.529) (width 0.5) (layer "B.Cu") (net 3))
 (segment (start 80.264 69.723) (end 81.661 71.12) (width 0.5) (layer "B.Cu") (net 3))
 (segment (start 83.058 71.12) (end 84.435 72.497) (width 0.5) (layer "B.Cu") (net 3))
 (segment (start 107.061 56.281) (end 107.061 39.243) (width 0.5) (layer "B.Cu") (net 3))
 (segment (start 87.376 39.624) (end 87.376 41.783) (width 0.5) (layer "B.Cu") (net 3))
 (segment (start 102.362 54.213189) (end 95.25 61.325189) (width 0.5) (layer "F.Cu") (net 16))
 (segment (start 102.362 43.307) (end 102.362 54.213189) (width 0.5) (layer "F.Cu") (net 16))
 (segment (start 95.25 61.325189) (end 95.25 73.533) (width 0.5) (layer "F.Cu") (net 16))
 (segment (start 95.25 73.533) (end 98.933 77.216) (width 0.5) (layer "F.Cu") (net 16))
 (segment (start 98.933 77.216) (end 99.314 77.216) (width 0.5) (layer "F.Cu") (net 16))
 (via (at 99.314 77.216) (size 1.8) (drill 0.3) (layers "F.Cu" "B.Cu") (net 16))
 (via (at 102.362 43.307) (size 1.8) (drill 0.3) (layers "F.Cu" "B.Cu") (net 16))
 (segment (start 104.013 40.386) (end 105.039 41.412) (width 0.5) (layer "B.Cu") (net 16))
 (segment (start 100.584 40.386) (end 104.013 40.386) (width 0.5) (layer "B.Cu") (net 16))
 (segment (start 98.552 77.978) (end 99.314 77.216) (width 0.5) (layer "B.Cu") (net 16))
 (segment (start 87.249 44.724) (end 91.349 44.724) (width 0.5) (layer "B.Cu") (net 16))
 (segment (start 100.584 40.386) (end 100.584 42.021) (width 0.5) (layer "B.Cu") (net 16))
 (segment (start 105.039 43.063) (end 102.606 43.063) (width 0.5) (layer "B.Cu") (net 16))
 (segment (start 91.365 44.74) (end 97.865 44.74) (width 0.5) (layer "B.Cu") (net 16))
 (segment (start 91.349 44.724) (end 91.365 44.74) (width 0.5) (layer "B.Cu") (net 16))
 (segment (start 100.584 42.021) (end 97.865 44.74) (width 0.5) (layer "B.Cu") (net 16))
 (segment (start 102.606 43.063) (end 102.362 43.307) (width 0.5) (layer "B.Cu") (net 16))
 (segment (start 95.377 77.978) (end 98.552 77.978) (width 0.5) (layer "B.Cu") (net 16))
 (segment (start 105.039 41.412) (end 105.039 43.063) (width 0.5) (layer "B.Cu") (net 16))
 (segment (start 89.916 39.624) (end 89.916 38.227) (width 0.5) (layer "B.Cu") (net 1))
 (segment (start 91.44 36.703) (end 108.331 36.703) (width 0.5) (layer "B.Cu") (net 1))
 (segment (start 108.331 36.703) (end 110.49 38.862) (width 0.5) (layer "B.Cu") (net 1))
 (segment (start 89.916 38.227) (end 91.44 36.703) (width 0.5) (layer "B.Cu") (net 1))
 (segment (start 112.659 71.003) (end 114.036 71.003) (width 0.5) (layer "B.Cu") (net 13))
 (segment (start 118.872 80.264) (end 119.634 79.502) (width 0.5) (layer "B.Cu") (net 13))
 (segment (start 90.805 80.264) (end 118.872 80.264) (width 0.5) (layer "B.Cu") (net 13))
 (segment (start 115.316 69.723) (end 117.475 69.723) (width 0.5) (layer "B.Cu") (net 13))
 (segment (start 90.297 79.756) (end 90.805 80.264) (width 0.5) (layer "B.Cu") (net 13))
 (segment (start 118.872 69.723) (end 117.475 69.723) (width 0.5) (layer "B.Cu") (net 13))
 (segment (start 119.634 70.485) (end 118.872 69.723) (width 0.5) (layer "B.Cu") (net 13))
 (segment (start 119.634 79.502) (end 119.634 70.485) (width 0.5) (layer "B.Cu") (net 13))
 (segment (start 114.036 71.003) (end 115.316 69.723) (width 0.5) (layer "B.Cu") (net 13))
 (segment (start 90.297 77.978) (end 90.297 79.756) (width 0.5) (layer "B.Cu") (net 13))
 (segment (start 121.031 68.961) (end 121.031 80.645) (width 0.5) (layer "B.Cu") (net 14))
 (segment (start 87.757 79.629) (end 87.757 77.978) (width 0.5) (layer "B.Cu") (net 14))
 (segment (start 112.659 68.463) (end 113.655 68.463) (width 0.5) (layer "B.Cu") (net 14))
 (segment (start 114.935 67.183) (end 117.475 67.183) (width 0.5) (layer "B.Cu") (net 14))
 (segment (start 113.655 68.463) (end 114.935 67.183) (width 0.5) (layer "B.Cu") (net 14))
 (segment (start 117.475 67.183) (end 119.253 67.183) (width 0.5) (layer "B.Cu") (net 14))
 (segment (start 120.142 81.534) (end 89.662 81.534) (width 0.5) (layer "B.Cu") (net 14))
 (segment (start 119.253 67.183) (end 121.031 68.961) (width 0.5) (layer "B.Cu") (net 14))
 (segment (start 121.031 80.645) (end 120.142 81.534) (width 0.5) (layer "B.Cu") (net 14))
 (segment (start 89.662 81.534) (end 87.757 79.629) (width 0.5) (layer "B.Cu") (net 14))
 (segment (start 85.217 80.264) (end 85.217 77.978) (width 0.5) (layer "B.Cu") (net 15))
 (segment (start 112.659 65.923) (end 114.29 65.923) (width 0.5) (layer "B.Cu") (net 15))
 (segment (start 120.904 83.058) (end 88.011 83.058) (width 0.5) (layer "B.Cu") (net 15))
 (segment (start 122.682 81.28) (end 120.904 83.058) (width 0.5) (layer "B.Cu") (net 15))
 (segment (start 88.011 83.058) (end 85.217 80.264) (width 0.5) (layer "B.Cu") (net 15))
 (segment (start 122.682 67.31) (end 122.682 81.28) (width 0.5) (layer "B.Cu") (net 15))
 (segment (start 114.29 65.923) (end 115.57 64.643) (width 0.5) (layer "B.Cu") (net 15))
 (segment (start 115.57 64.643) (end 117.475 64.643) (width 0.5) (layer "B.Cu") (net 15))
 (segment (start 117.475 64.643) (end 120.015 64.643) (width 0.5) (layer "B.Cu") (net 15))
 (segment (start 120.015 64.643) (end 122.682 67.31) (width 0.5) (layer "B.Cu") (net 15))
 (segment (start 85.232 49.291) (end 87.503 51.562) (width 0.5) (layer "B.Cu") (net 17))
 (segment (start 99.695 51.562) (end 100.203 51.054) (width 0.5) (layer "B.Cu") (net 17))
 (segment (start 87.503 51.562) (end 99.695 51.562) (width 0.5) (layer "B.Cu") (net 17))
 (segment (start 100.203 46.482) (end 101.082 45.603) (width 0.5) (layer "B.Cu") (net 17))
 (segment (start 101.082 45.603) (end 105.039 45.603) (width 0.5) (layer "B.Cu") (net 17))
 (segment (start 82.677 49.291) (end 85.232 49.291) (width 0.5) (layer "B.Cu") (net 17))
 (segment (start 100.203 51.054) (end 100.203 46.482) (width 0.5) (layer "B.Cu") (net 17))
 (segment (start 100.203 52.959) (end 101.854 51.308) (width 0.5) (layer "B.Cu") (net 18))
 (segment (start 82.677 51.831) (end 85.105 51.831) (width 0.5) (layer "B.Cu") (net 18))
 (segment (start 85.105 51.831) (end 86.233 52.959) (width 0.5) (layer "B.Cu") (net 18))
 (segment (start 101.854 51.308) (end 101.854 48.641) (width 0.5) (layer "B.Cu") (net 18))
 (segment (start 86.233 52.959) (end 100.203 52.959) (width 0.5) (layer "B.Cu") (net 18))
 (segment (start 101.854 48.641) (end 102.352 48.143) (width 0.5) (layer "B.Cu") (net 18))
 (segment (start 102.352 48.143) (end 105.039 48.143) (width 0.5) (layer "B.Cu") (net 18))
 (segment (start 82.677 54.371) (end 100.823 54.371) (width 0.5) (layer "B.Cu") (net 19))
 (segment (start 104.511 50.683) (end 105.039 50.683) (width 0.5) (layer "B.Cu") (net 19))
 (segment (start 100.823 54.371) (end 104.511 50.683) (width 0.5) (layer "B.Cu") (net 19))
 (segment (start 101.346 56.134) (end 86.36 56.134) (width 0.5) (layer "B.Cu") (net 20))
 (segment (start 86.36 56.134) (end 85.583 56.911) (width 0.5) (layer "B.Cu") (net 20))
 (segment (start 85.583 56.911) (end 82.677 56.911) (width 0.5) (layer "B.Cu") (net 20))
 (segment (start 105.039 53.223) (end 104.257 53.223) (width 0.5) (layer "B.Cu") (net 20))
 (segment (start 104.257 53.223) (end 101.346 56.134) (width 0.5) (layer "B.Cu") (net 20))
 (segment (start 102.235 57.785) (end 104.257 55.763) (width 0.5) (layer "B.Cu") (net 21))
 (segment (start 104.257 55.763) (end 105.039 55.763) (width 0.5) (layer "B.Cu") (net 21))
 (segment (start 86.995 57.785) (end 102.235 57.785) (width 0.5) (layer "B.Cu") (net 21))
 (segment (start 85.329 59.451) (end 86.995 57.785) (width 0.5) (layer "B.Cu") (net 21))
 (segment (start 82.677 59.451) (end 85.329 59.451) (width 0.5) (layer "B.Cu") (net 21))
 (segment (start 87.264 61.991) (end 82.677 61.991) (width 0.5) (layer "B.Cu") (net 22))
 (segment (start 88.9 63.627) (end 87.264 61.991) (width 0.5) (layer "B.Cu") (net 22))
 (segment (start 105.039 68.463) (end 102.479 68.463) (width 0.5) (layer "B.Cu") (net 22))
 (segment (start 88.9 70.485) (end 88.9 63.627) (width 0.5) (layer "B.Cu") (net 22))
 (segment (start 89.789 71.374) (end 88.9 70.485) (width 0.5) (layer "B.Cu") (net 22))
 (segment (start 99.568 71.374) (end 89.789 71.374) (width 0.5) (layer "B.Cu") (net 22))
 (segment (start 102.479 68.463) (end 99.568 71.374) (width 0.5) (layer "B.Cu") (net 22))
 (segment (start 82.677 64.531) (end 85.486 64.531) (width 0.5) (layer "B.Cu") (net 23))
 (segment (start 103.622 71.003) (end 105.039 71.003) (width 0.5) (layer "B.Cu") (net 23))
 (segment (start 85.486 64.531) (end 87.122 66.167) (width 0.5) (layer "B.Cu") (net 23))
 (segment (start 87.122 71.247) (end 88.773 72.898) (width 0.5) (layer "B.Cu") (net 23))
 (segment (start 87.122 66.167) (end 87.122 71.247) (width 0.5) (layer "B.Cu") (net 23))
 (segment (start 88.773 72.898) (end 101.727 72.898) (width 0.5) (layer "B.Cu") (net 23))
 (segment (start 101.727 72.898) (end 103.622 71.003) (width 0.5) (layer "B.Cu") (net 23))
 (segment (start 84.597 67.071) (end 85.852 68.326) (width 0.5) (layer "B.Cu") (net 24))
 (segment (start 104.16 74.422) (end 105.039 73.543) (width 0.5) (layer "B.Cu") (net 24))
 (segment (start 82.677 67.071) (end 84.597 67.071) (width 0.5) (layer "B.Cu") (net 24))
 (segment (start 85.852 72.263) (end 88.011 74.422) (width 0.5) (layer "B.Cu") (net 24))
 (segment (start 88.011 74.422) (end 104.16 74.422) (width 0.5) (layer "B.Cu") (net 24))
 (segment (start 85.852 68.326) (end 85.852 72.263) (width 0.5) (layer "B.Cu") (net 24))
 (segment (start 105.039 76.083) (end 106.69 76.083) (width 0.5) (layer "B.Cu") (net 10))
 (segment (start 106.69 76.083) (end 108.839 78.232) (width 0.5) (layer "B.Cu") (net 10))
 (segment (start 114.808 78.232) (end 115.697 77.343) (width 0.5) (layer "B.Cu") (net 10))
 (segment (start 108.839 78.232) (end 114.808 78.232) (width 0.5) (layer "B.Cu") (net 10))
 (segment (start 115.697 77.343) (end 117.475 77.343) (width 0.5) (layer "B.Cu") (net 10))
 (segment (start 112.659 76.083) (end 113.909 76.083) (width 0.5) (layer "B.Cu") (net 11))
 (segment (start 115.189 74.803) (end 117.475 74.803) (width 0.5) (layer "B.Cu") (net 11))
 (segment (start 113.909 76.083) (end 115.189 74.803) (width 0.5) (layer "B.Cu") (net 11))
 (segment (start 115.189 72.263) (end 117.475 72.263) (width 0.5) (layer "B.Cu") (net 12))
 (segment (start 112.659 73.543) (end 113.909 73.543) (width 0.5) (layer "B.Cu") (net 12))
 (segment (start 113.909 73.543) (end 115.189 72.263) (width 0.5) (layer "B.Cu") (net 12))
 (segment (start 112.659 55.763) (end 117.465 55.763) (width 0.5) (layer "B.Cu") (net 4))
 (segment (start 117.465 55.763) (end 117.475 55.753) (width 0.5) (layer "B.Cu") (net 4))
 (segment (start 112.659 53.223) (end 117.465 53.223) (width 0.5) (layer "B.Cu") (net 5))
 (segment (start 117.465 53.223) (end 117.475 53.213) (width 0.5) (layer "B.Cu") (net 5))
 (segment (start 117.465 50.683) (end 117.475 50.673) (width 0.5) (layer "B.Cu") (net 6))
 (segment (start 112.659 50.683) (end 117.465 50.683) (width 0.5) (layer "B.Cu") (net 6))
 (segment (start 112.659 48.143) (end 117.465 48.143) (width 0.5) (layer "B.Cu") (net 7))
 (segment (start 117.465 48.143) (end 117.475 48.133) (width 0.5) (layer "B.Cu") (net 7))
 (segment (start 112.659 45.603) (end 117.465 45.603) (width 0.5) (layer "B.Cu") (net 8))
 (segment (start 117.465 45.603) (end 117.475 45.593) (width 0.5) (layer "B.Cu") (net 8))
 (segment (start 117.465 43.063) (end 117.475 43.053) (width 0.5) (layer "B.Cu") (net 9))
 (segment (start 112.659 43.063) (end 117.465 43.063) (width 0.5) (layer "B.Cu") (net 9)))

